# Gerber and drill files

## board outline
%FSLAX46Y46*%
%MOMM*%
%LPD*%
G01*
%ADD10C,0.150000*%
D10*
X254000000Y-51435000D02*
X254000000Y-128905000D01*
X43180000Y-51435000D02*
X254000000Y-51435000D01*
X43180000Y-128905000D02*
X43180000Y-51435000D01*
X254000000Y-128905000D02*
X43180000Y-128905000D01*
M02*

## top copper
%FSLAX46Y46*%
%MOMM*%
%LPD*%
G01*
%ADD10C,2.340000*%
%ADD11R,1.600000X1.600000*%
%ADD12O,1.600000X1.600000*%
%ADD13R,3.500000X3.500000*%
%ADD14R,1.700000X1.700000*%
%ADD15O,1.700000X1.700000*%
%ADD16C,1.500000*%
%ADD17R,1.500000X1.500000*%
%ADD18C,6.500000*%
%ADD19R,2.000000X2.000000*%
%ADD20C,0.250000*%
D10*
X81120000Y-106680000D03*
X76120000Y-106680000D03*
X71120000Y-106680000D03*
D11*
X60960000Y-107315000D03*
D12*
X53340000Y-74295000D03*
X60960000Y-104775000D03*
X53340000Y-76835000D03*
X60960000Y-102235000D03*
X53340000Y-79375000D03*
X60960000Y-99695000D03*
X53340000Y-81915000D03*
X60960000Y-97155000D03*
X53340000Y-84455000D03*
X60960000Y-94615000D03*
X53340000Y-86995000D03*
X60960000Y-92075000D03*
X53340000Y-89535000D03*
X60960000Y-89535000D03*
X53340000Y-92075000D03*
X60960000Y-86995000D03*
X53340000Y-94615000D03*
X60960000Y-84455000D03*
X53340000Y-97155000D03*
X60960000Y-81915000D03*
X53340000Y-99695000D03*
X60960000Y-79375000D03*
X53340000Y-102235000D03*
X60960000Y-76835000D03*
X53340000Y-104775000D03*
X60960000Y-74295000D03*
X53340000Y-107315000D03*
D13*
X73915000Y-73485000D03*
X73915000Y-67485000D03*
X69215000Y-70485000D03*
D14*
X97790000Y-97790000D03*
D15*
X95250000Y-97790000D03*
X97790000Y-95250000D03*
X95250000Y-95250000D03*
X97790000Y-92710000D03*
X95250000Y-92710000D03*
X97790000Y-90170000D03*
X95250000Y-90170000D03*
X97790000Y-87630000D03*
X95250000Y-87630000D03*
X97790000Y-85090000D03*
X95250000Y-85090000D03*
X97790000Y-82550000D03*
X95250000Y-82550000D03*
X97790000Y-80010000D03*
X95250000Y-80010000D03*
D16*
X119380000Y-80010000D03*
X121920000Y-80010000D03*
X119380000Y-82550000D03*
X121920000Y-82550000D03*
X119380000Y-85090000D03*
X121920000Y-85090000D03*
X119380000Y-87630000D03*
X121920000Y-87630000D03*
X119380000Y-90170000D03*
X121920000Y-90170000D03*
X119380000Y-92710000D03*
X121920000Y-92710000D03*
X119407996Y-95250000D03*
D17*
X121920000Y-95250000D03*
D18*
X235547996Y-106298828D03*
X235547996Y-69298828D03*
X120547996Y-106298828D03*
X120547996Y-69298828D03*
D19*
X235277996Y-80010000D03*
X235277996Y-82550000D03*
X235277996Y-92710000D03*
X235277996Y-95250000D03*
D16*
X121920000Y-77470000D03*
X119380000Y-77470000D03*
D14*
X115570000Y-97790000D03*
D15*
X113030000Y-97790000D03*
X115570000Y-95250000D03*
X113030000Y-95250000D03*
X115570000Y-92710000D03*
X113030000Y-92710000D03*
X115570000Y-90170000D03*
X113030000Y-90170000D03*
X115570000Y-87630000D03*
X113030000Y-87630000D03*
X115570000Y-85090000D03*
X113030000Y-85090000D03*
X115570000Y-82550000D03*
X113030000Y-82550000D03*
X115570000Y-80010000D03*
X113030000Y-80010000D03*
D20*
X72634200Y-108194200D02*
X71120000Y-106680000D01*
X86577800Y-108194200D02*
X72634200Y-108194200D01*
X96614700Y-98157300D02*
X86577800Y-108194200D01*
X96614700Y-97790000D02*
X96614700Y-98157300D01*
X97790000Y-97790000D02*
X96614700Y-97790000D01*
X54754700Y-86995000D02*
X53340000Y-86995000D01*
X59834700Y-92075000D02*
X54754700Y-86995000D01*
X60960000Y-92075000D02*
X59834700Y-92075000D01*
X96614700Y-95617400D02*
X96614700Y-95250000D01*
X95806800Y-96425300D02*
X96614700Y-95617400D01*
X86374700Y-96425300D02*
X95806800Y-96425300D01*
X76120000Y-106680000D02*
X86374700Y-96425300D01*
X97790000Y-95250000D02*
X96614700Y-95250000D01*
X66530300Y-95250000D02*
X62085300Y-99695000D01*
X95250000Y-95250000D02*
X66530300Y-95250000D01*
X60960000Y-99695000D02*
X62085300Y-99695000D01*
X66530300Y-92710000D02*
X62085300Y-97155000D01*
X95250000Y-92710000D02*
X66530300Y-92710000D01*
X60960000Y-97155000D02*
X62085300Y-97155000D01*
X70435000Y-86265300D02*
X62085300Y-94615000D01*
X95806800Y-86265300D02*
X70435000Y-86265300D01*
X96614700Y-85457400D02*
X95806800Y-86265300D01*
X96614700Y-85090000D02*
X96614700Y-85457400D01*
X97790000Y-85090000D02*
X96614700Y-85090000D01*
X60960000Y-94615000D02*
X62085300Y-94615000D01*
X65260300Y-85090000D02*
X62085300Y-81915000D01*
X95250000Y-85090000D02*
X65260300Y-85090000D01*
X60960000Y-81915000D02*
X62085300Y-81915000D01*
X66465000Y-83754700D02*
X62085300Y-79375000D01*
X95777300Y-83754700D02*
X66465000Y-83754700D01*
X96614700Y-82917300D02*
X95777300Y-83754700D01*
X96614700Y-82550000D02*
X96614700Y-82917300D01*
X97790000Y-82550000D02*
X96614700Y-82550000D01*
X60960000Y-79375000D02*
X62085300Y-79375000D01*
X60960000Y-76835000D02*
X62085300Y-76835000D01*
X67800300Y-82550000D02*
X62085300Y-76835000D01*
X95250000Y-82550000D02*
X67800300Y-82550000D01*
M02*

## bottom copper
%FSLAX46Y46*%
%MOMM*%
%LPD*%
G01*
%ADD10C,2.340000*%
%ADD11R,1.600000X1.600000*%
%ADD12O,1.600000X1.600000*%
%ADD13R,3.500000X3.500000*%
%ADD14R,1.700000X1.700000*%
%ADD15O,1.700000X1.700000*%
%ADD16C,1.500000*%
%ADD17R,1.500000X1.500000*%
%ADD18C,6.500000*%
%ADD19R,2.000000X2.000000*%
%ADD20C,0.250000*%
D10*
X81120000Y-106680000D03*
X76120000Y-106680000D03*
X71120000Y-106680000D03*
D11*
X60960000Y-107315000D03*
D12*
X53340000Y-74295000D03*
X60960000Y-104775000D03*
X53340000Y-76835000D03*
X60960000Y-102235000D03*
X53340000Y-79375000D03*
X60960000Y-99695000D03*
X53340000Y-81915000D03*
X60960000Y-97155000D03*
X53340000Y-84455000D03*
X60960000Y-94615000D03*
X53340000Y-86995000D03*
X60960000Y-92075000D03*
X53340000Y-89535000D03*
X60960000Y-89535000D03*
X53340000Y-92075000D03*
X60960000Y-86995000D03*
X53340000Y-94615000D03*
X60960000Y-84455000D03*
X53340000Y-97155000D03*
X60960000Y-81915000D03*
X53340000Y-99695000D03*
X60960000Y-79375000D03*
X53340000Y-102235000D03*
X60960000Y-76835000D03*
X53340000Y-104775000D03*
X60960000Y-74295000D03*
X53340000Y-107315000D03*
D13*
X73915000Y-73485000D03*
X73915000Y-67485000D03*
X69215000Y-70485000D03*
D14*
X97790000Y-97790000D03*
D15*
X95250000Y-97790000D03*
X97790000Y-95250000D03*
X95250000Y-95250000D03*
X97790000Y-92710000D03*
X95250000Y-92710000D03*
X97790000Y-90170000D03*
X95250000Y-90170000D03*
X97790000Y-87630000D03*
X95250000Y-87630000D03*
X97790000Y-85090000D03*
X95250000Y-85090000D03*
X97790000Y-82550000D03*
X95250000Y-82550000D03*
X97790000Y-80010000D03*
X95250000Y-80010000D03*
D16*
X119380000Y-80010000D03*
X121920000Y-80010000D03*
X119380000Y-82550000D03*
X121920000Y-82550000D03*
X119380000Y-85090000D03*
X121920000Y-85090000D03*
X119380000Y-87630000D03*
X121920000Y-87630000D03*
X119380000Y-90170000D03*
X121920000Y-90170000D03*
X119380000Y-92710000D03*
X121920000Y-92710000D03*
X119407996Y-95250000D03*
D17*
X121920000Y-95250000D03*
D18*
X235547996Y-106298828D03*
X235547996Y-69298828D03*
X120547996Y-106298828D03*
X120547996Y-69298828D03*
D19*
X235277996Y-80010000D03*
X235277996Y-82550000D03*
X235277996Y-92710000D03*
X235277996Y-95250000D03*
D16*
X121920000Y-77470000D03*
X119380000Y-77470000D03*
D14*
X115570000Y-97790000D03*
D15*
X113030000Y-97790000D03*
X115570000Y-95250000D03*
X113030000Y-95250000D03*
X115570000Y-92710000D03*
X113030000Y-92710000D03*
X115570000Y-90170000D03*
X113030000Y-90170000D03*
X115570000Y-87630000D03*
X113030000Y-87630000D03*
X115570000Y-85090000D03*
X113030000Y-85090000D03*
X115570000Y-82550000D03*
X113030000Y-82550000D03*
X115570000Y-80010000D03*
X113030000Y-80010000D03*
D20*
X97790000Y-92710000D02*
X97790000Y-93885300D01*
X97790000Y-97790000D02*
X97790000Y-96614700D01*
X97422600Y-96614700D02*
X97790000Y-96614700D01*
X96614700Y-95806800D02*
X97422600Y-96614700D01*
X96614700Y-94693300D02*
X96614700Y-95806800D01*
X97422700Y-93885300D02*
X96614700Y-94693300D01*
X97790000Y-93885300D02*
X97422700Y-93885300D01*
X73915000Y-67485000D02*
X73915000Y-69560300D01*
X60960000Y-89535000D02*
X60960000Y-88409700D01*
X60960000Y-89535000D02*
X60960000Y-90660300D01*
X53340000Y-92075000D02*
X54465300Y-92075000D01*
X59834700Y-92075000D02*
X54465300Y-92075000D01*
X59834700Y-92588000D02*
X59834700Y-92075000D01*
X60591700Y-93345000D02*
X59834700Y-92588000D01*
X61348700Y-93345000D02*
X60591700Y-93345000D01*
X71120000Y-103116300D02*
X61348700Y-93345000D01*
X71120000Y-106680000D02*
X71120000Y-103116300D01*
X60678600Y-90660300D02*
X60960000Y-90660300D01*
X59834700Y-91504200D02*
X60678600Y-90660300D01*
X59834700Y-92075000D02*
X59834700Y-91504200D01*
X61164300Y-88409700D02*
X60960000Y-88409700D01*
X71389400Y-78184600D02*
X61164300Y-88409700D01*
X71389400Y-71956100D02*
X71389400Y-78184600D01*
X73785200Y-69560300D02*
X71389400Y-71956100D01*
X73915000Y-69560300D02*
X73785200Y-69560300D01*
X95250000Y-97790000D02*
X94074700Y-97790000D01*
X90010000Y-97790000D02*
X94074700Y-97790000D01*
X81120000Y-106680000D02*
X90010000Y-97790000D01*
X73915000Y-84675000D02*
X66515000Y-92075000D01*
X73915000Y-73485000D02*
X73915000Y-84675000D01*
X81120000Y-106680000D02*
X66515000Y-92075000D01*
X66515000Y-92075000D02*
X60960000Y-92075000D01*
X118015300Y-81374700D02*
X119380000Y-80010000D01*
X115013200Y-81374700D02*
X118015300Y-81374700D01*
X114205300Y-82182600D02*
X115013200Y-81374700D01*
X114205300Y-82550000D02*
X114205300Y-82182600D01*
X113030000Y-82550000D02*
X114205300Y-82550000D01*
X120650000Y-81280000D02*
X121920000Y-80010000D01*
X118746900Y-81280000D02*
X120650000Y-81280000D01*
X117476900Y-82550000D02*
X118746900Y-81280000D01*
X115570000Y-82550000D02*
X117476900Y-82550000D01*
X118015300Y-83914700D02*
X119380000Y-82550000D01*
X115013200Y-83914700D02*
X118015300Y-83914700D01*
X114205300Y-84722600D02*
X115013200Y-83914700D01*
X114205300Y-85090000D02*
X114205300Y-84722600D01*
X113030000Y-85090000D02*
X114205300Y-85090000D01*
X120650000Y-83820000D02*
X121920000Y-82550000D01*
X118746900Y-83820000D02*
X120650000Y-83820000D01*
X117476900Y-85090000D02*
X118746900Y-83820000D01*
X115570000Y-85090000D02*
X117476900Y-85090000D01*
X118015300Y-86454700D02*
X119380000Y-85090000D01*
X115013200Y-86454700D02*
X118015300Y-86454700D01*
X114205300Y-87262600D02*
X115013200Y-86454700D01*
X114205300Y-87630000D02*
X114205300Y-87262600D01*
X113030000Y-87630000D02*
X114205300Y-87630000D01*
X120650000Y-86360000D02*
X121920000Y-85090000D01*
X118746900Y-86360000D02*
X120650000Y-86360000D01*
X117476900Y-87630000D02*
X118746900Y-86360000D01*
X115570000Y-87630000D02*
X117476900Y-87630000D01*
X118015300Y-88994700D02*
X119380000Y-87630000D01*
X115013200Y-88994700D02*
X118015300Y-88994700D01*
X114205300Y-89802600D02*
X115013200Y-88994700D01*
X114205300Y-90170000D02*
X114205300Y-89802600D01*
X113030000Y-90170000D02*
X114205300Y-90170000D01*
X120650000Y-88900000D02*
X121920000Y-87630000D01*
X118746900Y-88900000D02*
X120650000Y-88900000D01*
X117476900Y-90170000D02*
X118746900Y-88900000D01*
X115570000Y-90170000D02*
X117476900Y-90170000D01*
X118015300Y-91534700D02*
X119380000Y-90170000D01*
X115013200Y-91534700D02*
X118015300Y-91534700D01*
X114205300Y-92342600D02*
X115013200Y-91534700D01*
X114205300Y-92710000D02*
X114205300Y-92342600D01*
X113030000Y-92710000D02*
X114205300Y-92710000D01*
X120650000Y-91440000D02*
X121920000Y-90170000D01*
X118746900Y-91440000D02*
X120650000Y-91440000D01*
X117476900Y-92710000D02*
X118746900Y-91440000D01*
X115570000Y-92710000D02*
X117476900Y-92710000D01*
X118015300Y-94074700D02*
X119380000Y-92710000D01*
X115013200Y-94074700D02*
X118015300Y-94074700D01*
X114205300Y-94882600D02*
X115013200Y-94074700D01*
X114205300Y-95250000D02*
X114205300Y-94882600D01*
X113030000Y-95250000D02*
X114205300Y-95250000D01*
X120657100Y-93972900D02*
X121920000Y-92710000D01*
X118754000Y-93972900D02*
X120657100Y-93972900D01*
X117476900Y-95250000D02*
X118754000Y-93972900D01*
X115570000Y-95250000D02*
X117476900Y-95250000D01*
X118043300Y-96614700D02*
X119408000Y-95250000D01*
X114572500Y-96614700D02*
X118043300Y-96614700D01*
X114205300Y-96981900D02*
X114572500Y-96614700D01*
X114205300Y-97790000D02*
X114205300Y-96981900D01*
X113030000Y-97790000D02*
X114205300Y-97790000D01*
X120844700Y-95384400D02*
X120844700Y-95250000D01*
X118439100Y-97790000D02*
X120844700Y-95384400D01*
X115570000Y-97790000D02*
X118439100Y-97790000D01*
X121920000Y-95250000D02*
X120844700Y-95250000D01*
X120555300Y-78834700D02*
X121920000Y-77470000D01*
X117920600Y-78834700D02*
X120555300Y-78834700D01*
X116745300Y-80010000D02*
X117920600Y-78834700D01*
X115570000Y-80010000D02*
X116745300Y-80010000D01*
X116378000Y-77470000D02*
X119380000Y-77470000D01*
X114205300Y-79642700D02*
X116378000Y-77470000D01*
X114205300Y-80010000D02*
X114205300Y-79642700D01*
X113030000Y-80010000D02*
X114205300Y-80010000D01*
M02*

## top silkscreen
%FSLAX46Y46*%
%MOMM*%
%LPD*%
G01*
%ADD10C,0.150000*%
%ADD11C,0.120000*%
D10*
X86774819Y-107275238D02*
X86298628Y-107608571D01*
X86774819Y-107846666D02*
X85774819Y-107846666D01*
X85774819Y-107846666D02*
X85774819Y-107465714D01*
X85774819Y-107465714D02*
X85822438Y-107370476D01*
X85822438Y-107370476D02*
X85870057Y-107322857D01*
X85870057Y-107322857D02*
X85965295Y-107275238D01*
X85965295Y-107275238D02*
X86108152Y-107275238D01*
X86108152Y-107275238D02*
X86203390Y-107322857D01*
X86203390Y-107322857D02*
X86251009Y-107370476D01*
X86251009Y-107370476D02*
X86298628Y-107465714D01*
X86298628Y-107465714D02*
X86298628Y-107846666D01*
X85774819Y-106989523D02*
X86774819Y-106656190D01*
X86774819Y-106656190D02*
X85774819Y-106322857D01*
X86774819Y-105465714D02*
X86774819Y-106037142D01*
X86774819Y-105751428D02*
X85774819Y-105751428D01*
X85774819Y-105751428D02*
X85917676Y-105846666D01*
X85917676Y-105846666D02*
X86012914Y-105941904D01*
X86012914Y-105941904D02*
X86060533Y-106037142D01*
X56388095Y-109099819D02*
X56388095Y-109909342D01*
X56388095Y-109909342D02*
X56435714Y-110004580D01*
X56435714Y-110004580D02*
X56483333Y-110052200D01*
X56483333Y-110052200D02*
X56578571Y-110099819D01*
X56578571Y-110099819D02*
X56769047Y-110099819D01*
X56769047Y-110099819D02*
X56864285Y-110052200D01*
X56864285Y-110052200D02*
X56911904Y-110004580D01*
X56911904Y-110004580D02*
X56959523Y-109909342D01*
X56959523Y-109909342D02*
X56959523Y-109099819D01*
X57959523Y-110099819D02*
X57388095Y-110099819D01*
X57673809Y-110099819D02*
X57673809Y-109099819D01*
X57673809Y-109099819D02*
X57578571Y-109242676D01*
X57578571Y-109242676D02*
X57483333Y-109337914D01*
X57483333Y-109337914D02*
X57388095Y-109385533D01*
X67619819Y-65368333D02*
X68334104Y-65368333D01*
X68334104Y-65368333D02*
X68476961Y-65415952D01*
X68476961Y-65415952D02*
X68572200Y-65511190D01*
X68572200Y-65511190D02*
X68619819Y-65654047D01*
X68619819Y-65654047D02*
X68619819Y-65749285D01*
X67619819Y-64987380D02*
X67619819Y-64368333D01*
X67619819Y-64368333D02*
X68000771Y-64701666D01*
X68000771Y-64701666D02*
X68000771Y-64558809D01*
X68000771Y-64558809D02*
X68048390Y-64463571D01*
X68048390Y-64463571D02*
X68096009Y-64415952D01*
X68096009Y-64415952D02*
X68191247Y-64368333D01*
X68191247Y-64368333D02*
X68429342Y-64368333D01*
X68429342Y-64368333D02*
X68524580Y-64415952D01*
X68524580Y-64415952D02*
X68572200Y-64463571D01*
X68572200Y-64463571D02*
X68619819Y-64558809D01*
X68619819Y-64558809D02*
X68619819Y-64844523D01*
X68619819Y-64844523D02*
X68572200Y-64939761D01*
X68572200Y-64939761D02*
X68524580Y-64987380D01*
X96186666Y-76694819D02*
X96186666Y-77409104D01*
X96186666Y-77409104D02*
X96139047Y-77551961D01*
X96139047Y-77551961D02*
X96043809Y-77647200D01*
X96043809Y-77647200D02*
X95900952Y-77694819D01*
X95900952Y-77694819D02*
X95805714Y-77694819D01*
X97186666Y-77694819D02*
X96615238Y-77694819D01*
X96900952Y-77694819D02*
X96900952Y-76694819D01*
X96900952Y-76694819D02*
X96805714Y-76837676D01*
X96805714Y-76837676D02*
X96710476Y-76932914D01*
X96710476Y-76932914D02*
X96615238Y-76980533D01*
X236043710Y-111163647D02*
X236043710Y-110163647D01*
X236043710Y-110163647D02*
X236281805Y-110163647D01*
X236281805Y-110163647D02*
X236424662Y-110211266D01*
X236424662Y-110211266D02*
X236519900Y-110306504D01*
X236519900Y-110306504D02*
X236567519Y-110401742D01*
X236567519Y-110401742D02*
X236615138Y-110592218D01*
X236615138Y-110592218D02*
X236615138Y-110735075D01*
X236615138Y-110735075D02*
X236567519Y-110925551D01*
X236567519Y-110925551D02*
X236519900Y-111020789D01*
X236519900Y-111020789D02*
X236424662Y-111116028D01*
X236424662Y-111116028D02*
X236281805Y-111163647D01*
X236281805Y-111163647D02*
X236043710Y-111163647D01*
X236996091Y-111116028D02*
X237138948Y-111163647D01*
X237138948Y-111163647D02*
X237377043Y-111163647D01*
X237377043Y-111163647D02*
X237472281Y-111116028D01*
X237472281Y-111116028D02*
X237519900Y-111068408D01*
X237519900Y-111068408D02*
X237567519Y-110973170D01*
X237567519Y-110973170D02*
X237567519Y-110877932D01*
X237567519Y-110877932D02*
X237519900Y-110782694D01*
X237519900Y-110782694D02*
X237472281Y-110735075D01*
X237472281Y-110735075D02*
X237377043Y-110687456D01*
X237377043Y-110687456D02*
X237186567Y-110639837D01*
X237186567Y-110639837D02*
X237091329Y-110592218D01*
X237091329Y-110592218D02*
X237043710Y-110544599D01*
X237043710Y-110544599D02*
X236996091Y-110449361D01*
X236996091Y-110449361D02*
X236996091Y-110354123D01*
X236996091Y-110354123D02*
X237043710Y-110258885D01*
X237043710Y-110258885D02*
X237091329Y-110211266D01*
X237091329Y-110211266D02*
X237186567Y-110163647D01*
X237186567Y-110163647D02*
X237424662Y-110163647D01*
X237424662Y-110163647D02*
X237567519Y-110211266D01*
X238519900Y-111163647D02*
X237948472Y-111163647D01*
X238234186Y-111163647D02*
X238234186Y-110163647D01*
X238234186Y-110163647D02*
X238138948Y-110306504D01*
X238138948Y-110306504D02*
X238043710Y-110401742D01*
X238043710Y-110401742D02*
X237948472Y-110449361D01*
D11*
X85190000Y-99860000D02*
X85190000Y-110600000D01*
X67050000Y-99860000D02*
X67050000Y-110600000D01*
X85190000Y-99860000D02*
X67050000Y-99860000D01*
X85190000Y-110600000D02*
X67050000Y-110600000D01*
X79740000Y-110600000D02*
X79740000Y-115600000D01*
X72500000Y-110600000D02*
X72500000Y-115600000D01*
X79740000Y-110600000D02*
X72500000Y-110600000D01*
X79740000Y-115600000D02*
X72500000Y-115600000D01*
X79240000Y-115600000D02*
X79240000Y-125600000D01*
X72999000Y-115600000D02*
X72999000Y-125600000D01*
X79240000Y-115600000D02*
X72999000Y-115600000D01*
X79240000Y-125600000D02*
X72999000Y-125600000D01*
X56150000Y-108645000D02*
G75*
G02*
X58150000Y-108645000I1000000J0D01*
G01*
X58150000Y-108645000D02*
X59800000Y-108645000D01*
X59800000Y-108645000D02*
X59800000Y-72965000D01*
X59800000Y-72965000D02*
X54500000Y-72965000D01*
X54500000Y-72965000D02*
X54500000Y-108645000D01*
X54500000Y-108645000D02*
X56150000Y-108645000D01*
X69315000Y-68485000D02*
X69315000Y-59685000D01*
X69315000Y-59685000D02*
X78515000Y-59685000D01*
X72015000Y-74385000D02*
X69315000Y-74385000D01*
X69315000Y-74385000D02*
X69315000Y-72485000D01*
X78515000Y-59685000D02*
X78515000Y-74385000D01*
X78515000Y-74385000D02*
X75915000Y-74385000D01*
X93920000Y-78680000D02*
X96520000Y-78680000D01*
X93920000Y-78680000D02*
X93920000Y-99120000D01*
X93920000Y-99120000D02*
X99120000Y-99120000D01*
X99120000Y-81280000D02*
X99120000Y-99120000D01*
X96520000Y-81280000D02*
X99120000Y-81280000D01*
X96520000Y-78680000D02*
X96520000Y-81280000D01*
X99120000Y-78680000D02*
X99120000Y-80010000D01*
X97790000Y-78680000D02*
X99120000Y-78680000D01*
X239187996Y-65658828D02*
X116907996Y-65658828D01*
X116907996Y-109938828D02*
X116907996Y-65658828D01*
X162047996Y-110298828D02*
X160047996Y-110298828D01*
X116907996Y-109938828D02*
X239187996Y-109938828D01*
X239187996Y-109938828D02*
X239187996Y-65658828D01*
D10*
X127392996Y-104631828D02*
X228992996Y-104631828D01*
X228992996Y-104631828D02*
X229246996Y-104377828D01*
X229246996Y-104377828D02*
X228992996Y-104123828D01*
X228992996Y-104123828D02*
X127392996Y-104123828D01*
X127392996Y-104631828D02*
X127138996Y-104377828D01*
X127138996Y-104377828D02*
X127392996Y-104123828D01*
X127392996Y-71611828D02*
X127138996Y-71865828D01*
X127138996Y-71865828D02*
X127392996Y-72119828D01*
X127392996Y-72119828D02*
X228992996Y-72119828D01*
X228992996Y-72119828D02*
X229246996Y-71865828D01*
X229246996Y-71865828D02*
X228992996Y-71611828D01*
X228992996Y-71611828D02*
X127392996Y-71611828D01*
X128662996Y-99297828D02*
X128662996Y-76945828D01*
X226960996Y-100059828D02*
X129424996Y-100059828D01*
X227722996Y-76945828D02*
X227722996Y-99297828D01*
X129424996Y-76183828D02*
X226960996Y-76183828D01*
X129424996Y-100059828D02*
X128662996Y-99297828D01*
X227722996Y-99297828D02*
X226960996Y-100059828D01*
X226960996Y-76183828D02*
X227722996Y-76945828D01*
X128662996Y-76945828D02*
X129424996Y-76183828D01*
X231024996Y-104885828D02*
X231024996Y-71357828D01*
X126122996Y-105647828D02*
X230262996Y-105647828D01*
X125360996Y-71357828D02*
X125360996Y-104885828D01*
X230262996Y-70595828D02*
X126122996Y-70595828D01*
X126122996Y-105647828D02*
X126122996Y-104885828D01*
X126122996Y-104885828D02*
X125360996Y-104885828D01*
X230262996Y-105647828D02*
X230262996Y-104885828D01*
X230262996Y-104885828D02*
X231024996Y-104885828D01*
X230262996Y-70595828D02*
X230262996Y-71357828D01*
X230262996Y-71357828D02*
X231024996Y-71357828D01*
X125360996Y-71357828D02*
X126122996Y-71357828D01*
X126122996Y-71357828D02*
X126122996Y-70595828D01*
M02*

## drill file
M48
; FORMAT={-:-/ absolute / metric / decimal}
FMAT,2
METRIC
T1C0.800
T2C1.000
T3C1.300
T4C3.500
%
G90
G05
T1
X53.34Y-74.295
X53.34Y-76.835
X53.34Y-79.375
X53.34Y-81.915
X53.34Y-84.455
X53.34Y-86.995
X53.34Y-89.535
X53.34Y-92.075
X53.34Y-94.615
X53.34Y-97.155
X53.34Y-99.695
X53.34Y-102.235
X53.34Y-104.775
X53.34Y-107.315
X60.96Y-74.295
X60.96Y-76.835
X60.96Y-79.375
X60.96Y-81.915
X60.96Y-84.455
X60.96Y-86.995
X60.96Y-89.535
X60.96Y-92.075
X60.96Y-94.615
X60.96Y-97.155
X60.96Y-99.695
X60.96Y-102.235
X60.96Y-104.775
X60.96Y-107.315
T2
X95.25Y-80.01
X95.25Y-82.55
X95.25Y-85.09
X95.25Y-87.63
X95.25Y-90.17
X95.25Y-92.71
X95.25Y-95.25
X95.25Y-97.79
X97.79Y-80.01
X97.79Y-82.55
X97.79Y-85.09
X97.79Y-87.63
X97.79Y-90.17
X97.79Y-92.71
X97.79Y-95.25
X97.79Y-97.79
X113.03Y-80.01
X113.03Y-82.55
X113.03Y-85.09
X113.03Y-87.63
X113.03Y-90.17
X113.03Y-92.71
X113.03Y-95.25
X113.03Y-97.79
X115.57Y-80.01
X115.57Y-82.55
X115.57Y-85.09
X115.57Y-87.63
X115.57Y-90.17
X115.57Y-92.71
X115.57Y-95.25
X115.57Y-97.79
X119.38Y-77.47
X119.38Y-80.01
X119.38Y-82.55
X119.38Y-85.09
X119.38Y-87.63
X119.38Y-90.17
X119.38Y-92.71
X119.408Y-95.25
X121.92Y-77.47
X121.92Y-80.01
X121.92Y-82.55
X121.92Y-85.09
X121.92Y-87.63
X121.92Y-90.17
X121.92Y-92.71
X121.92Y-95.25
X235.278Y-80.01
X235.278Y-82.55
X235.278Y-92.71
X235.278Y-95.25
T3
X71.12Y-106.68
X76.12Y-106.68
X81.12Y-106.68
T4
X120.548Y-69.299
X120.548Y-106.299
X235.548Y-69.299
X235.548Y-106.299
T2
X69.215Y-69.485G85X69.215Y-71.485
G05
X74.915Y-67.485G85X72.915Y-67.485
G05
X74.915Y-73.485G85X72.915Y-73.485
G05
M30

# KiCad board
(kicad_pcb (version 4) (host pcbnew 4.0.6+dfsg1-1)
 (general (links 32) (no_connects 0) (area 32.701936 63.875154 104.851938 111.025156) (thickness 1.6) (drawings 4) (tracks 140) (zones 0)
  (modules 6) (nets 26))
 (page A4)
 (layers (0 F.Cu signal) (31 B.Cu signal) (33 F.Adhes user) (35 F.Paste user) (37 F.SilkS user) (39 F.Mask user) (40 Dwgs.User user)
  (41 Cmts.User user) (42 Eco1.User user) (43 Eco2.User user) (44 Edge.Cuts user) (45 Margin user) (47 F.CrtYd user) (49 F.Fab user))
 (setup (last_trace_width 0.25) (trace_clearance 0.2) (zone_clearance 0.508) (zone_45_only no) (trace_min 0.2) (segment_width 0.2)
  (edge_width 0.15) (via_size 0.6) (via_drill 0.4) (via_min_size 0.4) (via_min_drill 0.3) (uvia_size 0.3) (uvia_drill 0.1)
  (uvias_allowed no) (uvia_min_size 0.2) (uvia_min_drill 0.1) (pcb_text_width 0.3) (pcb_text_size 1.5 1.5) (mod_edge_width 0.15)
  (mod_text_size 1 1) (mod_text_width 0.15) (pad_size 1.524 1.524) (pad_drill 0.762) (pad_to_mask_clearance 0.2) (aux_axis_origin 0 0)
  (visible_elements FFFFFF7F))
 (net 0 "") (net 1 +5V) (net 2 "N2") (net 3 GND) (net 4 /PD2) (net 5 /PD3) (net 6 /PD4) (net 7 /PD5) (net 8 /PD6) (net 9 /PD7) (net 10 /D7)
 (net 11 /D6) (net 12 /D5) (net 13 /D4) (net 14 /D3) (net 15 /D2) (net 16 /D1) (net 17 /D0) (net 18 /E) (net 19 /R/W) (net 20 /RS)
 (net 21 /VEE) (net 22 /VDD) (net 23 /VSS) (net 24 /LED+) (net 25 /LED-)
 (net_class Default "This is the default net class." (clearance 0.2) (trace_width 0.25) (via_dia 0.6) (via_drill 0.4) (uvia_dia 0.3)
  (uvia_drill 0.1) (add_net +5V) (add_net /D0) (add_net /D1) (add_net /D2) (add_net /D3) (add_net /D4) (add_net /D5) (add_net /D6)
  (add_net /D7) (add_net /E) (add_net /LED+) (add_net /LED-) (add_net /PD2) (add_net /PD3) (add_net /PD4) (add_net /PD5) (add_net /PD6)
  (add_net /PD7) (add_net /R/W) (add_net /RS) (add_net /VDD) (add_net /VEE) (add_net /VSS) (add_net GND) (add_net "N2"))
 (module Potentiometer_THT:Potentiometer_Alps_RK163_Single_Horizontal (layer F.Cu) (at 71.12 106.68 270)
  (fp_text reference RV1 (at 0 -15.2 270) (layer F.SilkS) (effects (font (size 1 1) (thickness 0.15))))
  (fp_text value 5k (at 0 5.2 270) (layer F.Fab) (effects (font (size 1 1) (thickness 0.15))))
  (fp_line (start -6.82 -14.07) (end 3.92 -14.07) (layer F.SilkS) (width 0.12))
  (fp_line (start -6.82 4.07) (end 3.92 4.07) (layer F.SilkS) (width 0.12))
  (fp_line (start -6.82 -14.07) (end -6.82 4.07) (layer F.SilkS) (width 0.12))
  (fp_line (start 3.92 -14.07) (end 3.92 4.07) (layer F.SilkS) (width 0.12))
  (fp_line (start 3.92 -8.62) (end 8.92 -8.62) (layer F.SilkS) (width 0.12))
  (fp_line (start 3.92 -1.38) (end 8.92 -1.38) (layer F.SilkS) (width 0.12))
  (fp_line (start 3.92 -8.62) (end 3.92 -1.38) (layer F.SilkS) (width 0.12))
  (fp_line (start 8.92 -8.62) (end 8.92 -1.38) (layer F.SilkS) (width 0.12))
  (fp_line (start 8.92 -8.12) (end 18.92 -8.12) (layer F.SilkS) (width 0.12))
  (fp_line (start 8.92 -1.879) (end 18.92 -1.879) (layer F.SilkS) (width 0.12))
  (fp_line (start 8.92 -8.12) (end 8.92 -1.879) (layer F.SilkS) (width 0.12))
  (fp_line (start 18.92 -8.12) (end 18.92 -1.879) (layer F.SilkS) (width 0.12))
  (pad 3 thru_hole circle (at 0 -10 270) (size 2.34 2.34) (drill 1.3) (layers *.Cu *.Mask) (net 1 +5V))
  (pad 2 thru_hole circle (at 0 -5 270) (size 2.34 2.34) (drill 1.3) (layers *.Cu *.Mask) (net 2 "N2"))
  (pad 1 thru_hole circle (at 0 0 270) (size 2.34 2.34) (drill 1.3) (layers *.Cu *.Mask) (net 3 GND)))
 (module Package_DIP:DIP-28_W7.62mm (layer F.Cu) (at 60.96 107.315 180)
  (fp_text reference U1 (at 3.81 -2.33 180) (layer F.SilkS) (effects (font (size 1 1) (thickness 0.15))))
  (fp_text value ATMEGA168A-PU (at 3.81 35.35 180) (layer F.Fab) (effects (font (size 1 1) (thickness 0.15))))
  (fp_arc (start 3.81 -1.33) (end 2.81 -1.33) (angle -180) (layer F.SilkS) (width 0.12))
  (fp_line (start 2.81 -1.33) (end 1.16 -1.33) (layer F.SilkS) (width 0.12))
  (fp_line (start 1.16 -1.33) (end 1.16 34.35) (layer F.SilkS) (width 0.12))
  (fp_line (start 1.16 34.35) (end 6.46 34.35) (layer F.SilkS) (width 0.12))
  (fp_line (start 6.46 34.35) (end 6.46 -1.33) (layer F.SilkS) (width 0.12))
  (fp_line (start 6.46 -1.33) (end 4.81 -1.33) (layer F.SilkS) (width 0.12))
  (pad 1 thru_hole rect (at 0 0 180) (size 1.6 1.6) (drill 0.8) (layers *.Cu *.Mask))
  (pad 15 thru_hole oval (at 7.62 33.02 180) (size 1.6 1.6) (drill 0.8) (layers *.Cu *.Mask))
  (pad 2 thru_hole oval (at 0 2.54 180) (size 1.6 1.6) (drill 0.8) (layers *.Cu *.Mask))
  (pad 16 thru_hole oval (at 7.62 30.48 180) (size 1.6 1.6) (drill 0.8) (layers *.Cu *.Mask))
  (pad 3 thru_hole oval (at 0 5.08 180) (size 1.6 1.6) (drill 0.8) (layers *.Cu *.Mask))
  (pad 17 thru_hole oval (at 7.62 27.94 180) (size 1.6 1.6) (drill 0.8) (layers *.Cu *.Mask))
  (pad 4 thru_hole oval (at 0 7.62 180) (size 1.6 1.6) (drill 0.8) (layers *.Cu *.Mask) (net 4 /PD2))
  (pad 18 thru_hole oval (at 7.62 25.4 180) (size 1.6 1.6) (drill 0.8) (layers *.Cu *.Mask))
  (pad 5 thru_hole oval (at 0 10.16 180) (size 1.6 1.6) (drill 0.8) (layers *.Cu *.Mask) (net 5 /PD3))
  (pad 19 thru_hole oval (at 7.62 22.86 180) (size 1.6 1.6) (drill 0.8) (layers *.Cu *.Mask))
  (pad 6 thru_hole oval (at 0 12.7 180) (size 1.6 1.6) (drill 0.8) (layers *.Cu *.Mask) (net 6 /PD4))
  (pad 20 thru_hole oval (at 7.62 20.32 180) (size 1.6 1.6) (drill 0.8) (layers *.Cu *.Mask) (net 1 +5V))
  (pad 7 thru_hole oval (at 0 15.24 180) (size 1.6 1.6) (drill 0.8) (layers *.Cu *.Mask) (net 1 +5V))
  (pad 21 thru_hole oval (at 7.62 17.78 180) (size 1.6 1.6) (drill 0.8) (layers *.Cu *.Mask))
  (pad 8 thru_hole oval (at 0 17.78 180) (size 1.6 1.6) (drill 0.8) (layers *.Cu *.Mask) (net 3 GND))
  (pad 22 thru_hole oval (at 7.62 15.24 180) (size 1.6 1.6) (drill 0.8) (layers *.Cu *.Mask) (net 3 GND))
  (pad 9 thru_hole oval (at 0 20.32 180) (size 1.6 1.6) (drill 0.8) (layers *.Cu *.Mask))
  (pad 23 thru_hole oval (at 7.62 12.7 180) (size 1.6 1.6) (drill 0.8) (layers *.Cu *.Mask))
  (pad 10 thru_hole oval (at 0 22.86 180) (size 1.6 1.6) (drill 0.8) (layers *.Cu *.Mask))
  (pad 24 thru_hole oval (at 7.62 10.16 180) (size 1.6 1.6) (drill 0.8) (layers *.Cu *.Mask))
  (pad 11 thru_hole oval (at 0 25.4 180) (size 1.6 1.6) (drill 0.8) (layers *.Cu *.Mask) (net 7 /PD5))
  (pad 25 thru_hole oval (at 7.62 7.62 180) (size 1.6 1.6) (drill 0.8) (layers *.Cu *.Mask))
  (pad 12 thru_hole oval (at 0 27.94 180) (size 1.6 1.6) (drill 0.8) (layers *.Cu *.Mask) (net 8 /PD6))
  (pad 26 thru_hole oval (at 7.62 5.08 180) (size 1.6 1.6) (drill 0.8) (layers *.Cu *.Mask))
  (pad 13 thru_hole oval (at 0 30.48 180) (size 1.6 1.6) (drill 0.8) (layers *.Cu *.Mask) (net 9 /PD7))
  (pad 27 thru_hole oval (at 7.62 2.54 180) (size 1.6 1.6) (drill 0.8) (layers *.Cu *.Mask))
  (pad 14 thru_hole oval (at 0 33.02 180) (size 1.6 1.6) (drill 0.8) (layers *.Cu *.Mask))
  (pad 28 thru_hole oval (at 7.62 0 180) (size 1.6 1.6) (drill 0.8) (layers *.Cu *.Mask)))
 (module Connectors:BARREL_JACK (layer F.Cu) (at 73.915 73.485 270)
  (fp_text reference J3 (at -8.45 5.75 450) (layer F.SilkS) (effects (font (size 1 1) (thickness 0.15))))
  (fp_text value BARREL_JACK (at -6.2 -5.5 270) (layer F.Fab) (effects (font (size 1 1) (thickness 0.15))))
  (fp_line (start -5 4.6) (end -13.8 4.6) (layer F.SilkS) (width 0.12))
  (fp_line (start -13.8 4.6) (end -13.8 -4.6) (layer F.SilkS) (width 0.12))
  (fp_line (start 0.9 1.9) (end 0.9 4.6) (layer F.SilkS) (width 0.12))
  (fp_line (start 0.9 4.6) (end -1 4.6) (layer F.SilkS) (width 0.12))
  (fp_line (start -13.8 -4.6) (end 0.9 -4.6) (layer F.SilkS) (width 0.12))
  (fp_line (start 0.9 -4.6) (end 0.9 -2) (layer F.SilkS) (width 0.12))
  (pad 1 thru_hole rect (at 0 0 270) (size 3.5 3.5) (drill oval 1 3) (layers *.Cu *.Mask) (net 1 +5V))
  (pad 2 thru_hole rect (at -6 0 270) (size 3.5 3.5) (drill oval 1 3) (layers *.Cu *.Mask) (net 3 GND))
  (pad 3 thru_hole rect (at -3 4.7 270) (size 3.5 3.5) (drill oval 3 1) (layers *.Cu *.Mask)))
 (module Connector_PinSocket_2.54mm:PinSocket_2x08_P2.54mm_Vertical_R (layer F.Cu) (at 97.79 80.01)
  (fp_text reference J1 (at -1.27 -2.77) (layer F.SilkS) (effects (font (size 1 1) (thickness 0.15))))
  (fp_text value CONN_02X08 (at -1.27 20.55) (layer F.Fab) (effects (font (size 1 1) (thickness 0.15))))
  (fp_line (start -3.87 -1.33) (end -1.27 -1.33) (layer F.SilkS) (width 0.12))
  (fp_line (start -3.87 -1.33) (end -3.87 19.11) (layer F.SilkS) (width 0.12))
  (fp_line (start -3.87 19.11) (end 1.33 19.11) (layer F.SilkS) (width 0.12))
  (fp_line (start 1.33 1.27) (end 1.33 19.11) (layer F.SilkS) (width 0.12))
  (fp_line (start -1.27 1.27) (end 1.33 1.27) (layer F.SilkS) (width 0.12))
  (fp_line (start -1.27 -1.33) (end -1.27 1.27) (layer F.SilkS) (width 0.12))
  (fp_line (start 1.33 -1.33) (end 1.33 0) (layer F.SilkS) (width 0.12))
  (fp_line (start 0 -1.33) (end 1.33 -1.33) (layer F.SilkS) (width 0.12))
  (pad 1 thru_hole rect (at 0 17.78) (size 1.7 1.7) (drill 1) (layers *.Cu *.Mask) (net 3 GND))
  (pad 2 thru_hole oval (at -2.54 17.78) (size 1.7 1.7) (drill 1) (layers *.Cu *.Mask) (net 1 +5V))
  (pad 3 thru_hole oval (at 0 15.24) (size 1.7 1.7) (drill 1) (layers *.Cu *.Mask) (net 2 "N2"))
  (pad 4 thru_hole oval (at -2.54 15.24) (size 1.7 1.7) (drill 1) (layers *.Cu *.Mask) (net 4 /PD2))
  (pad 5 thru_hole oval (at 0 12.7) (size 1.7 1.7) (drill 1) (layers *.Cu *.Mask) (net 3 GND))
  (pad 6 thru_hole oval (at -2.54 12.7) (size 1.7 1.7) (drill 1) (layers *.Cu *.Mask) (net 5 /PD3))
  (pad 7 thru_hole oval (at 0 10.16) (size 1.7 1.7) (drill 1) (layers *.Cu *.Mask))
  (pad 8 thru_hole oval (at -2.54 10.16) (size 1.7 1.7) (drill 1) (layers *.Cu *.Mask))
  (pad 9 thru_hole oval (at 0 7.62) (size 1.7 1.7) (drill 1) (layers *.Cu *.Mask))
  (pad 10 thru_hole oval (at -2.54 7.62) (size 1.7 1.7) (drill 1) (layers *.Cu *.Mask))
  (pad 11 thru_hole oval (at 0 5.08) (size 1.7 1.7) (drill 1) (layers *.Cu *.Mask) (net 6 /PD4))
  (pad 12 thru_hole oval (at -2.54 5.08) (size 1.7 1.7) (drill 1) (layers *.Cu *.Mask) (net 7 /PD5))
  (pad 13 thru_hole oval (at 0 2.54) (size 1.7 1.7) (drill 1) (layers *.Cu *.Mask) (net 8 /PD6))
  (pad 14 thru_hole oval (at -2.54 2.54) (size 1.7 1.7) (drill 1) (layers *.Cu *.Mask) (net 9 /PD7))
  (pad 15 thru_hole oval (at 0 0) (size 1.7 1.7) (drill 1) (layers *.Cu *.Mask))
  (pad 16 thru_hole oval (at -2.54 0) (size 1.7 1.7) (drill 1) (layers *.Cu *.Mask)))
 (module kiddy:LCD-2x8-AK (layer F.Cu) (at 177.8 87.63)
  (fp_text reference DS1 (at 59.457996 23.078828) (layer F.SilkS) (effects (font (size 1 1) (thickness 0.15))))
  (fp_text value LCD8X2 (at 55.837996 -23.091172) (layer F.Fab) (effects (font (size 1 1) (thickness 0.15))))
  (fp_line (start 61.387996 -21.971172) (end -60.892004 -21.971172) (layer F.SilkS) (width 0.12))
  (fp_line (start -60.892004 22.308828) (end -60.892004 -21.971172) (layer F.SilkS) (width 0.12))
  (fp_line (start -15.752004 22.668828) (end -17.752004 22.668828) (layer F.SilkS) (width 0.12))
  (fp_line (start -60.892004 22.308828) (end 61.387996 22.308828) (layer F.SilkS) (width 0.12))
  (fp_line (start 61.387996 22.308828) (end 61.387996 -21.971172) (layer F.SilkS) (width 0.12))
  (fp_line (start -50.407004 17.001828) (end 51.192996 17.001828) (layer F.SilkS) (width 0.15))
  (fp_line (start 51.192996 17.001828) (end 51.446996 16.747828) (layer F.SilkS) (width 0.15))
  (fp_line (start 51.446996 16.747828) (end 51.192996 16.493828) (layer F.SilkS) (width 0.15))
  (fp_line (start 51.192996 16.493828) (end -50.407004 16.493828) (layer F.SilkS) (width 0.15))
  (fp_line (start -50.407004 17.001828) (end -50.661004 16.747828) (layer F.SilkS) (width 0.15))
  (fp_line (start -50.661004 16.747828) (end -50.407004 16.493828) (layer F.SilkS) (width 0.15))
  (fp_line (start -50.407004 -16.018172) (end -50.661004 -15.764172) (layer F.SilkS) (width 0.15))
  (fp_line (start -50.661004 -15.764172) (end -50.407004 -15.510172) (layer F.SilkS) (width 0.15))
  (fp_line (start -50.407004 -15.510172) (end 51.192996 -15.510172) (layer F.SilkS) (width 0.15))
  (fp_line (start 51.192996 -15.510172) (end 51.446996 -15.764172) (layer F.SilkS) (width 0.15))
  (fp_line (start 51.446996 -15.764172) (end 51.192996 -16.018172) (layer F.SilkS) (width 0.15))
  (fp_line (start 51.192996 -16.018172) (end -50.407004 -16.018172) (layer F.SilkS) (width 0.15))
  (fp_line (start -49.137004 11.667828) (end -49.137004 -10.684172) (layer F.SilkS) (width 0.15))
  (fp_line (start 49.160996 12.429828) (end -48.375004 12.429828) (layer F.SilkS) (width 0.15))
  (fp_line (start 49.922996 -10.684172) (end 49.922996 11.667828) (layer F.SilkS) (width 0.15))
  (fp_line (start -48.375004 -11.446172) (end 49.160996 -11.446172) (layer F.SilkS) (width 0.15))
  (fp_line (start -48.375004 12.429828) (end -49.137004 11.667828) (layer F.SilkS) (width 0.15))
  (fp_line (start 49.922996 11.667828) (end 49.160996 12.429828) (layer F.SilkS) (width 0.15))
  (fp_line (start 49.160996 -11.446172) (end 49.922996 -10.684172) (layer F.SilkS) (width 0.15))
  (fp_line (start -49.137004 -10.684172) (end -48.375004 -11.446172) (layer F.SilkS) (width 0.15))
  (fp_line (start 53.224996 17.255828) (end 53.224996 -16.272172) (layer F.SilkS) (width 0.15))
  (fp_line (start -51.677004 18.017828) (end 52.462996 18.017828) (layer F.SilkS) (width 0.15))
  (fp_line (start -52.439004 -16.272172) (end -52.439004 17.255828) (layer F.SilkS) (width 0.15))
  (fp_line (start 52.462996 -17.034172) (end -51.677004 -17.034172) (layer F.SilkS) (width 0.15))
  (fp_line (start -51.677004 18.017828) (end -51.677004 17.255828) (layer F.SilkS) (width 0.15))
  (fp_line (start -51.677004 17.255828) (end -52.439004 17.255828) (layer F.SilkS) (width 0.15))
  (fp_line (start 52.462996 18.017828) (end 52.462996 17.255828) (layer F.SilkS) (width 0.15))
  (fp_line (start 52.462996 17.255828) (end 53.224996 17.255828) (layer F.SilkS) (width 0.15))
  (fp_line (start 52.462996 -17.034172) (end 52.462996 -16.272172) (layer F.SilkS) (width 0.15))
  (fp_line (start 52.462996 -16.272172) (end 53.224996 -16.272172) (layer F.SilkS) (width 0.15))
  (fp_line (start -52.439004 -16.272172) (end -51.677004 -16.272172) (layer F.SilkS) (width 0.15))
  (fp_line (start -51.677004 -16.272172) (end -51.677004 -17.034172) (layer F.SilkS) (width 0.15))
  (pad 14 thru_hole circle (at -58.42 -7.62 270) (size 1.5 1.5) (drill 1) (layers *.Cu *.Mask) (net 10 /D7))
  (pad 13 thru_hole circle (at -55.88 -7.62 270) (size 1.5 1.5) (drill 1) (layers *.Cu *.Mask) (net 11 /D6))
  (pad 12 thru_hole circle (at -58.42 -5.08 270) (size 1.5 1.5) (drill 1) (layers *.Cu *.Mask) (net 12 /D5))
  (pad 11 thru_hole circle (at -55.88 -5.08 270) (size 1.5 1.5) (drill 1) (layers *.Cu *.Mask) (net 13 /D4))
  (pad 10 thru_hole circle (at -58.42 -2.54 270) (size 1.5 1.5) (drill 1) (layers *.Cu *.Mask) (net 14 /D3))
  (pad 9 thru_hole circle (at -55.88 -2.54 270) (size 1.5 1.5) (drill 1) (layers *.Cu *.Mask) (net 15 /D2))
  (pad 8 thru_hole circle (at -58.42 0 270) (size 1.5 1.5) (drill 1) (layers *.Cu *.Mask) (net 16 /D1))
  (pad 7 thru_hole circle (at -55.88 0 270) (size 1.5 1.5) (drill 1) (layers *.Cu *.Mask) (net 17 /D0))
  (pad 6 thru_hole circle (at -58.42 2.54 270) (size 1.5 1.5) (drill 1) (layers *.Cu *.Mask) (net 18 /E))
  (pad 5 thru_hole circle (at -55.88 2.54 270) (size 1.5 1.5) (drill 1) (layers *.Cu *.Mask) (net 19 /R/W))
  (pad 4 thru_hole circle (at -58.42 5.08 270) (size 1.5 1.5) (drill 1) (layers *.Cu *.Mask) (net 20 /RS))
  (pad 3 thru_hole circle (at -55.88 5.08 270) (size 1.5 1.5) (drill 1) (layers *.Cu *.Mask) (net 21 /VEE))
  (pad 2 thru_hole circle (at -58.392004 7.62 90) (size 1.5 1.5) (drill 1) (layers *.Cu *.Mask) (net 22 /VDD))
  (pad 1 thru_hole rect (at -55.88 7.62 90) (size 1.5 1.5) (drill 1) (layers *.Cu *.Mask) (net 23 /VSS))
  (pad "" thru_hole circle (at 57.747996 18.668828) (size 6.5 6.5) (drill 3.5) (layers *.Cu *.Mask))
  (pad "" thru_hole circle (at 57.747996 -18.331172) (size 6.5 6.5) (drill 3.5) (layers *.Cu *.Mask))
  (pad "" thru_hole circle (at -57.252004 18.668828) (size 6.5 6.5) (drill 3.5) (layers *.Cu *.Mask))
  (pad "" thru_hole circle (at -57.252004 -18.331172) (size 6.5 6.5) (drill 3.5) (layers *.Cu *.Mask))
  (pad A1 thru_hole rect (at 57.477996 -7.62) (size 2 2) (drill 1) (layers *.Cu *.Mask))
  (pad K1 thru_hole rect (at 57.477996 -5.08) (size 2 2) (drill 1) (layers *.Cu *.Mask))
  (pad A2 thru_hole rect (at 57.477996 5.08) (size 2 2) (drill 1) (layers *.Cu *.Mask))
  (pad K2 thru_hole rect (at 57.477996 7.62) (size 2 2) (drill 1) (layers *.Cu *.Mask))
  (pad 15 thru_hole circle (at -55.88 -10.16 270) (size 1.5 1.5) (drill 1) (layers *.Cu *.Mask) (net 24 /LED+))
  (pad 16 thru_hole circle (at -58.42 -10.16 270) (size 1.5 1.5) (drill 1) (layers *.Cu *.Mask) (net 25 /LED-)))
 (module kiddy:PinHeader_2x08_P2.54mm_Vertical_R (layer B.Cu) (at 115.57 97.79 180)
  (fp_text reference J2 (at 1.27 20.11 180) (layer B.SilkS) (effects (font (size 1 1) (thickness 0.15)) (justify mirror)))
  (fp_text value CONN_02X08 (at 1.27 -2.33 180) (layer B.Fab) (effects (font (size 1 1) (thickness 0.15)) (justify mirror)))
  (pad 1 thru_hole rect (at 0 0 180) (size 1.7 1.7) (drill 1) (layers *.Cu *.Mask) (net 23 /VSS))
  (pad 2 thru_hole oval (at 2.54 0 180) (size 1.7 1.7) (drill 1) (layers *.Cu *.Mask) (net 22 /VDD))
  (pad 3 thru_hole oval (at 0 2.54 180) (size 1.7 1.7) (drill 1) (layers *.Cu *.Mask) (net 21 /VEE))
  (pad 4 thru_hole oval (at 2.54 2.54 180) (size 1.7 1.7) (drill 1) (layers *.Cu *.Mask) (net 20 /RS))
  (pad 5 thru_hole oval (at 0 5.08 180) (size 1.7 1.7) (drill 1) (layers *.Cu *.Mask) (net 19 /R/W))
  (pad 6 thru_hole oval (at 2.54 5.08 180) (size 1.7 1.7) (drill 1) (layers *.Cu *.Mask) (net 18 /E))
  (pad 7 thru_hole oval (at 0 7.62 180) (size 1.7 1.7) (drill 1) (layers *.Cu *.Mask) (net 17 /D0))
  (pad 8 thru_hole oval (at 2.54 7.62 180) (size 1.7 1.7) (drill 1) (layers *.Cu *.Mask) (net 16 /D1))
  (pad 9 thru_hole oval (at 0 10.16 180) (size 1.7 1.7) (drill 1) (layers *.Cu *.Mask) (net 15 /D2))
  (pad 10 thru_hole oval (at 2.54 10.16 180) (size 1.7 1.7) (drill 1) (layers *.Cu *.Mask) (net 14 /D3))
  (pad 11 thru_hole oval (at 0 12.7 180) (size 1.7 1.7) (drill 1) (layers *.Cu *.Mask) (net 13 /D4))
  (pad 12 thru_hole oval (at 2.54 12.7 180) (size 1.7 1.7) (drill 1) (layers *.Cu *.Mask) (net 12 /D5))
  (pad 13 thru_hole oval (at 0 15.24 180) (size 1.7 1.7) (drill 1) (layers *.Cu *.Mask) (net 11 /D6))
  (pad 14 thru_hole oval (at 2.54 15.24 180) (size 1.7 1.7) (drill 1) (layers *.Cu *.Mask) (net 10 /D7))
  (pad 15 thru_hole oval (at 0 17.78 180) (size 1.7 1.7) (drill 1) (layers *.Cu *.Mask) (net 24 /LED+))
  (pad 16 thru_hole oval (at 2.54 17.78 180) (size 1.7 1.7) (drill 1) (layers *.Cu *.Mask) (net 25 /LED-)))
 (gr_line (start 254 51.435) (end 254 128.905) (layer Edge.Cuts) (width 0.15))
 (gr_line (start 43.18 51.435) (end 254 51.435) (layer Edge.Cuts) (width 0.15))
 (gr_line (start 43.18 128.905) (end 43.18 51.435) (layer Edge.Cuts) (width 0.15))
 (gr_line (start 254 128.905) (end 43.18 128.905) (layer Edge.Cuts) (width 0.15))
 (segment (start 97.79 92.71) (end 97.79 93.8853) (width 0.25) (layer B.Cu) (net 3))
 (segment (start 97.79 97.79) (end 97.79 96.6147) (width 0.25) (layer B.Cu) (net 3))
 (segment (start 97.4226 96.6147) (end 97.79 96.6147) (width 0.25) (layer B.Cu) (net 3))
 (segment (start 96.6147 95.8068) (end 97.4226 96.6147) (width 0.25) (layer B.Cu) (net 3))
 (segment (start 96.6147 94.6933) (end 96.6147 95.8068) (width 0.25) (layer B.Cu) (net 3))
 (segment (start 97.4227 93.8853) (end 96.6147 94.6933) (width 0.25) (layer B.Cu) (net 3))
 (segment (start 97.79 93.8853) (end 97.4227 93.8853) (width 0.25) (layer B.Cu) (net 3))
 (segment (start 73.915 67.485) (end 73.915 69.5603) (width 0.25) (layer B.Cu) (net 3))
 (segment (start 60.96 89.535) (end 60.96 88.4097) (width 0.25) (layer B.Cu) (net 3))
 (segment (start 72.6342 108.1942) (end 71.12 106.68) (width 0.25) (layer F.Cu) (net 3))
 (segment (start 86.5778 108.1942) (end 72.6342 108.1942) (width 0.25) (layer F.Cu) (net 3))
 (segment (start 96.6147 98.1573) (end 86.5778 108.1942) (width 0.25) (layer F.Cu) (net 3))
 (segment (start 96.6147 97.79) (end 96.6147 98.1573) (width 0.25) (layer F.Cu) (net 3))
 (segment (start 97.79 97.79) (end 96.6147 97.79) (width 0.25) (layer F.Cu) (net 3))
 (segment (start 60.96 89.535) (end 60.96 90.6603) (width 0.25) (layer B.Cu) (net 3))
 (segment (start 53.34 92.075) (end 54.4653 92.075) (width 0.25) (layer B.Cu) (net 3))
 (segment (start 59.8347 92.075) (end 54.4653 92.075) (width 0.25) (layer B.Cu) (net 3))
 (segment (start 59.8347 92.588) (end 59.8347 92.075) (width 0.25) (layer B.Cu) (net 3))
 (segment (start 60.5917 93.345) (end 59.8347 92.588) (width 0.25) (layer B.Cu) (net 3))
 (segment (start 61.3487 93.345) (end 60.5917 93.345) (width 0.25) (layer B.Cu) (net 3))
 (segment (start 71.12 103.1163) (end 61.3487 93.345) (width 0.25) (layer B.Cu) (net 3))
 (segment (start 71.12 106.68) (end 71.12 103.1163) (width 0.25) (layer B.Cu) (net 3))
 (segment (start 60.6786 90.6603) (end 60.96 90.6603) (width 0.25) (layer B.Cu) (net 3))
 (segment (start 59.8347 91.5042) (end 60.6786 90.6603) (width 0.25) (layer B.Cu) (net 3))
 (segment (start 59.8347 92.075) (end 59.8347 91.5042) (width 0.25) (layer B.Cu) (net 3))
 (segment (start 61.1643 88.4097) (end 60.96 88.4097) (width 0.25) (layer B.Cu) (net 3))
 (segment (start 71.3894 78.1846) (end 61.1643 88.4097) (width 0.25) (layer B.Cu) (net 3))
 (segment (start 71.3894 71.9561) (end 71.3894 78.1846) (width 0.25) (layer B.Cu) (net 3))
 (segment (start 73.7852 69.5603) (end 71.3894 71.9561) (width 0.25) (layer B.Cu) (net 3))
 (segment (start 73.915 69.5603) (end 73.7852 69.5603) (width 0.25) (layer B.Cu) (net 3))
 (segment (start 54.7547 86.995) (end 53.34 86.995) (width 0.25) (layer F.Cu) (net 1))
 (segment (start 59.8347 92.075) (end 54.7547 86.995) (width 0.25) (layer F.Cu) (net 1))
 (segment (start 60.96 92.075) (end 59.8347 92.075) (width 0.25) (layer F.Cu) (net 1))
 (segment (start 95.25 97.79) (end 94.0747 97.79) (width 0.25) (layer B.Cu) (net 1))
 (segment (start 90.01 97.79) (end 94.0747 97.79) (width 0.25) (layer B.Cu) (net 1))
 (segment (start 81.12 106.68) (end 90.01 97.79) (width 0.25) (layer B.Cu) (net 1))
 (segment (start 73.915 84.675) (end 66.515 92.075) (width 0.25) (layer B.Cu) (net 1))
 (segment (start 73.915 73.485) (end 73.915 84.675) (width 0.25) (layer B.Cu) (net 1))
 (segment (start 81.12 106.68) (end 66.515 92.075) (width 0.25) (layer B.Cu) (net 1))
 (segment (start 66.515 92.075) (end 60.96 92.075) (width 0.25) (layer B.Cu) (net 1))
 (segment (start 96.6147 95.6174) (end 96.6147 95.25) (width 0.25) (layer F.Cu) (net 2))
 (segment (start 95.8068 96.4253) (end 96.6147 95.6174) (width 0.25) (layer F.Cu) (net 2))
 (segment (start 86.3747 96.4253) (end 95.8068 96.4253) (width 0.25) (layer F.Cu) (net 2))
 (segment (start 76.12 106.68) (end 86.3747 96.4253) (width 0.25) (layer F.Cu) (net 2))
 (segment (start 97.79 95.25) (end 96.6147 95.25) (width 0.25) (layer F.Cu) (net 2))
 (segment (start 66.5303 95.25) (end 62.0853 99.695) (width 0.25) (layer F.Cu) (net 4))
 (segment (start 95.25 95.25) (end 66.5303 95.25) (width 0.25) (layer F.Cu) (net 4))
 (segment (start 60.96 99.695) (end 62.0853 99.695) (width 0.25) (layer F.Cu) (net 4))
 (segment (start 66.5303 92.71) (end 62.0853 97.155) (width 0.25) (layer F.Cu) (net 5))
 (segment (start 95.25 92.71) (end 66.5303 92.71) (width 0.25) (layer F.Cu) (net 5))
 (segment (start 60.96 97.155) (end 62.0853 97.155) (width 0.25) (layer F.Cu) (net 5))
 (segment (start 70.435 86.2653) (end 62.0853 94.615) (width 0.25) (layer F.Cu) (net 6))
 (segment (start 95.8068 86.2653) (end 70.435 86.2653) (width 0.25) (layer F.Cu) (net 6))
 (segment (start 96.6147 85.4574) (end 95.8068 86.2653) (width 0.25) (layer F.Cu) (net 6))
 (segment (start 96.6147 85.09) (end 96.6147 85.4574) (width 0.25) (layer F.Cu) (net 6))
 (segment (start 97.79 85.09) (end 96.6147 85.09) (width 0.25) (layer F.Cu) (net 6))
 (segment (start 60.96 94.615) (end 62.0853 94.615) (width 0.25) (layer F.Cu) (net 6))
 (segment (start 65.2603 85.09) (end 62.0853 81.915) (width 0.25) (layer F.Cu) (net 7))
 (segment (start 95.25 85.09) (end 65.2603 85.09) (width 0.25) (layer F.Cu) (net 7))
 (segment (start 60.96 81.915) (end 62.0853 81.915) (width 0.25) (layer F.Cu) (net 7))
 (segment (start 66.465 83.7547) (end 62.0853 79.375) (width 0.25) (layer F.Cu) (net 8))
 (segment (start 95.7773 83.7547) (end 66.465 83.7547) (width 0.25) (layer F.Cu) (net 8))
 (segment (start 96.6147 82.9173) (end 95.7773 83.7547) (width 0.25) (layer F.Cu) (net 8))
 (segment (start 96.6147 82.55) (end 96.6147 82.9173) (width 0.25) (layer F.Cu) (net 8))
 (segment (start 97.79 82.55) (end 96.6147 82.55) (width 0.25) (layer F.Cu) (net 8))
 (segment (start 60.96 79.375) (end 62.0853 79.375) (width 0.25) (layer F.Cu) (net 8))
 (segment (start 60.96 76.835) (end 62.0853 76.835) (width 0.25) (layer F.Cu) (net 9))
 (segment (start 67.8003 82.55) (end 62.0853 76.835) (width 0.25) (layer F.Cu) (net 9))
 (segment (start 95.25 82.55) (end 67.8003 82.55) (width 0.25) (layer F.Cu) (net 9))
 (segment (start 118.0153 81.3747) (end 119.38 80.01) (width 0.25) (layer B.Cu) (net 10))
 (segment (start 115.0132 81.3747) (end 118.0153 81.3747) (width 0.25) (layer B.Cu) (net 10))
 (segment (start 114.2053 82.1826) (end 115.0132 81.3747) (width 0.25) (layer B.Cu) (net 10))
 (segment (start 114.2053 82.55) (end 114.2053 82.1826) (width 0.25) (layer B.Cu) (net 10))
 (segment (start 113.03 82.55) (end 114.2053 82.55) (width 0.25) (layer B.Cu) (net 10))
 (segment (start 120.65 81.28) (end 121.92 80.01) (width 0.25) (layer B.Cu) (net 11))
 (segment (start 118.7469 81.28) (end 120.65 81.28) (width 0.25) (layer B.Cu) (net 11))
 (segment (start 117.4769 82.55) (end 118.7469 81.28) (width 0.25) (layer B.Cu) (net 11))
 (segment (start 115.57 82.55) (end 117.4769 82.55) (width 0.25) (layer B.Cu) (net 11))
 (segment (start 118.0153 83.9147) (end 119.38 82.55) (width 0.25) (layer B.Cu) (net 12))
 (segment (start 115.0132 83.9147) (end 118.0153 83.9147) (width 0.25) (layer B.Cu) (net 12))
 (segment (start 114.2053 84.7226) (end 115.0132 83.9147) (width 0.25) (layer B.Cu) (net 12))
 (segment (start 114.2053 85.09) (end 114.2053 84.7226) (width 0.25) (layer B.Cu) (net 12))
 (segment (start 113.03 85.09) (end 114.2053 85.09) (width 0.25) (layer B.Cu) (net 12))
 (segment (start 120.65 83.82) (end 121.92 82.55) (width 0.25) (layer B.Cu) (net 13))
 (segment (start 118.7469 83.82) (end 120.65 83.82) (width 0.25) (layer B.Cu) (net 13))
 (segment (start 117.4769 85.09) (end 118.7469 83.82) (width 0.25) (layer B.Cu) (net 13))
 (segment (start 115.57 85.09) (end 117.4769 85.09) (width 0.25) (layer B.Cu) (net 13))
 (segment (start 118.0153 86.4547) (end 119.38 85.09) (width 0.25) (layer B.Cu) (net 14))
 (segment (start 115.0132 86.4547) (end 118.0153 86.4547) (width 0.25) (layer B.Cu) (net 14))
 (segment (start 114.2053 87.2626) (end 115.0132 86.4547) (width 0.25) (layer B.Cu) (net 14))
 (segment (start 114.2053 87.63) (end 114.2053 87.2626) (width 0.25) (layer B.Cu) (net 14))
 (segment (start 113.03 87.63) (end 114.2053 87.63) (width 0.25) (layer B.Cu) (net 14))
 (segment (start 120.65 86.36) (end 121.92 85.09) (width 0.25) (layer B.Cu) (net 15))
 (segment (start 118.7469 86.36) (end 120.65 86.36) (width 0.25) (layer B.Cu) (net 15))
 (segment (start 117.4769 87.63) (end 118.7469 86.36) (width 0.25) (layer B.Cu) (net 15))
 (segment (start 115.57 87.63) (end 117.4769 87.63) (width 0.25) (layer B.Cu) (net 15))
 (segment (start 118.0153 88.9947) (end 119.38 87.63) (width 0.25) (layer B.Cu) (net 16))
 (segment (start 115.0132 88.9947) (end 118.0153 88.9947) (width 0.25) (layer B.Cu) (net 16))
 (segment (start 114.2053 89.8026) (end 115.0132 88.9947) (width 0.25) (layer B.Cu) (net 16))
 (segment (start 114.2053 90.17) (end 114.2053 89.8026) (width 0.25) (layer B.Cu) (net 16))
 (segment (start 113.03 90.17) (end 114.2053 90.17) (width 0.25) (layer B.Cu) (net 16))
 (segment (start 120.65 88.9) (end 121.92 87.63) (width 0.25) (layer B.Cu) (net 17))
 (segment (start 118.7469 88.9) (end 120.65 88.9) (width 0.25) (layer B.Cu) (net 17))
 (segment (start 117.4769 90.17) (end 118.7469 88.9) (width 0.25) (layer B.Cu) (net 17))
 (segment (start 115.57 90.17) (end 117.4769 90.17) (width 0.25) (layer B.Cu) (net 17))
 (segment (start 118.0153 91.5347) (end 119.38 90.17) (width 0.25) (layer B.Cu) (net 18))
 (segment (start 115.0132 91.5347) (end 118.0153 91.5347) (width 0.25) (layer B.Cu) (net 18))
 (segment (start 114.2053 92.3426) (end 115.0132 91.5347) (width 0.25) (layer B.Cu) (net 18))
 (segment (start 114.2053 92.71) (end 114.2053 92.3426) (width 0.25) (layer B.Cu) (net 18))
 (segment (start 113.03 92.71) (end 114.2053 92.71) (width 0.25) (layer B.Cu) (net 18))
 (segment (start 120.65 91.44) (end 121.92 90.17) (width 0.25) (layer B.Cu) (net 19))
 (segment (start 118.7469 91.44) (end 120.65 91.44) (width 0.25) (layer B.Cu) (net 19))
 (segment (start 117.4769 92.71) (end 118.7469 91.44) (width 0.25) (layer B.Cu) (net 19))
 (segment (start 115.57 92.71) (end 117.4769 92.71) (width 0.25) (layer B.Cu) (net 19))
 (segment (start 118.0153 94.0747) (end 119.38 92.71) (width 0.25) (layer B.Cu) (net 20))
 (segment (start 115.0132 94.0747) (end 118.0153 94.0747) (width 0.25) (layer B.Cu) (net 20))
 (segment (start 114.2053 94.8826) (end 115.0132 94.0747) (width 0.25) (layer B.Cu) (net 20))
 (segment (start 114.2053 95.25) (end 114.2053 94.8826) (width 0.25) (layer B.Cu) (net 20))
 (segment (start 113.03 95.25) (end 114.2053 95.25) (width 0.25) (layer B.Cu) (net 20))
 (segment (start 120.6571 93.9729) (end 121.92 92.71) (width 0.25) (layer B.Cu) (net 21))
 (segment (start 118.754 93.9729) (end 120.6571 93.9729) (width 0.25) (layer B.Cu) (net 21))
 (segment (start 117.4769 95.25) (end 118.754 93.9729) (width 0.25) (layer B.Cu) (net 21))
 (segment (start 115.57 95.25) (end 117.4769 95.25) (width 0.25) (layer B.Cu) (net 21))
 (segment (start 118.0433 96.6147) (end 119.408 95.25) (width 0.25) (layer B.Cu) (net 22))
 (segment (start 114.5725 96.6147) (end 118.0433 96.6147) (width 0.25) (layer B.Cu) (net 22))
 (segment (start 114.2053 96.9819) (end 114.5725 96.6147) (width 0.25) (layer B.Cu) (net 22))
 (segment (start 114.2053 97.79) (end 114.2053 96.9819) (width 0.25) (layer B.Cu) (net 22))
 (segment (start 113.03 97.79) (end 114.2053 97.79) (width 0.25) (layer B.Cu) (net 22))
 (segment (start 120.8447 95.3844) (end 120.8447 95.25) (width 0.25) (layer B.Cu) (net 23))
 (segment (start 118.4391 97.79) (end 120.8447 95.3844) (width 0.25) (layer B.Cu) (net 23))
 (segment (start 115.57 97.79) (end 118.4391 97.79) (width 0.25) (layer B.Cu) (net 23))
 (segment (start 121.92 95.25) (end 120.8447 95.25) (width 0.25) (layer B.Cu) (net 23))
 (segment (start 120.5553 78.8347) (end 121.92 77.47) (width 0.25) (layer B.Cu) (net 24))
 (segment (start 117.9206 78.8347) (end 120.5553 78.8347) (width 0.25) (layer B.Cu) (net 24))
 (segment (start 116.7453 80.01) (end 117.9206 78.8347) (width 0.25) (layer B.Cu) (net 24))
 (segment (start 115.57 80.01) (end 116.7453 80.01) (width 0.25) (layer B.Cu) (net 24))
 (segment (start 116.378 77.47) (end 119.38 77.47) (width 0.25) (layer B.Cu) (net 25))
 (segment (start 114.2053 79.6427) (end 116.378 77.47) (width 0.25) (layer B.Cu) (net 25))
 (segment (start 114.2053 80.01) (end 114.2053 79.6427) (width 0.25) (layer B.Cu) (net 25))
 (segment (start 113.03 80.01) (end 114.2053 80.01) (width 0.25) (layer B.Cu) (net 25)))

